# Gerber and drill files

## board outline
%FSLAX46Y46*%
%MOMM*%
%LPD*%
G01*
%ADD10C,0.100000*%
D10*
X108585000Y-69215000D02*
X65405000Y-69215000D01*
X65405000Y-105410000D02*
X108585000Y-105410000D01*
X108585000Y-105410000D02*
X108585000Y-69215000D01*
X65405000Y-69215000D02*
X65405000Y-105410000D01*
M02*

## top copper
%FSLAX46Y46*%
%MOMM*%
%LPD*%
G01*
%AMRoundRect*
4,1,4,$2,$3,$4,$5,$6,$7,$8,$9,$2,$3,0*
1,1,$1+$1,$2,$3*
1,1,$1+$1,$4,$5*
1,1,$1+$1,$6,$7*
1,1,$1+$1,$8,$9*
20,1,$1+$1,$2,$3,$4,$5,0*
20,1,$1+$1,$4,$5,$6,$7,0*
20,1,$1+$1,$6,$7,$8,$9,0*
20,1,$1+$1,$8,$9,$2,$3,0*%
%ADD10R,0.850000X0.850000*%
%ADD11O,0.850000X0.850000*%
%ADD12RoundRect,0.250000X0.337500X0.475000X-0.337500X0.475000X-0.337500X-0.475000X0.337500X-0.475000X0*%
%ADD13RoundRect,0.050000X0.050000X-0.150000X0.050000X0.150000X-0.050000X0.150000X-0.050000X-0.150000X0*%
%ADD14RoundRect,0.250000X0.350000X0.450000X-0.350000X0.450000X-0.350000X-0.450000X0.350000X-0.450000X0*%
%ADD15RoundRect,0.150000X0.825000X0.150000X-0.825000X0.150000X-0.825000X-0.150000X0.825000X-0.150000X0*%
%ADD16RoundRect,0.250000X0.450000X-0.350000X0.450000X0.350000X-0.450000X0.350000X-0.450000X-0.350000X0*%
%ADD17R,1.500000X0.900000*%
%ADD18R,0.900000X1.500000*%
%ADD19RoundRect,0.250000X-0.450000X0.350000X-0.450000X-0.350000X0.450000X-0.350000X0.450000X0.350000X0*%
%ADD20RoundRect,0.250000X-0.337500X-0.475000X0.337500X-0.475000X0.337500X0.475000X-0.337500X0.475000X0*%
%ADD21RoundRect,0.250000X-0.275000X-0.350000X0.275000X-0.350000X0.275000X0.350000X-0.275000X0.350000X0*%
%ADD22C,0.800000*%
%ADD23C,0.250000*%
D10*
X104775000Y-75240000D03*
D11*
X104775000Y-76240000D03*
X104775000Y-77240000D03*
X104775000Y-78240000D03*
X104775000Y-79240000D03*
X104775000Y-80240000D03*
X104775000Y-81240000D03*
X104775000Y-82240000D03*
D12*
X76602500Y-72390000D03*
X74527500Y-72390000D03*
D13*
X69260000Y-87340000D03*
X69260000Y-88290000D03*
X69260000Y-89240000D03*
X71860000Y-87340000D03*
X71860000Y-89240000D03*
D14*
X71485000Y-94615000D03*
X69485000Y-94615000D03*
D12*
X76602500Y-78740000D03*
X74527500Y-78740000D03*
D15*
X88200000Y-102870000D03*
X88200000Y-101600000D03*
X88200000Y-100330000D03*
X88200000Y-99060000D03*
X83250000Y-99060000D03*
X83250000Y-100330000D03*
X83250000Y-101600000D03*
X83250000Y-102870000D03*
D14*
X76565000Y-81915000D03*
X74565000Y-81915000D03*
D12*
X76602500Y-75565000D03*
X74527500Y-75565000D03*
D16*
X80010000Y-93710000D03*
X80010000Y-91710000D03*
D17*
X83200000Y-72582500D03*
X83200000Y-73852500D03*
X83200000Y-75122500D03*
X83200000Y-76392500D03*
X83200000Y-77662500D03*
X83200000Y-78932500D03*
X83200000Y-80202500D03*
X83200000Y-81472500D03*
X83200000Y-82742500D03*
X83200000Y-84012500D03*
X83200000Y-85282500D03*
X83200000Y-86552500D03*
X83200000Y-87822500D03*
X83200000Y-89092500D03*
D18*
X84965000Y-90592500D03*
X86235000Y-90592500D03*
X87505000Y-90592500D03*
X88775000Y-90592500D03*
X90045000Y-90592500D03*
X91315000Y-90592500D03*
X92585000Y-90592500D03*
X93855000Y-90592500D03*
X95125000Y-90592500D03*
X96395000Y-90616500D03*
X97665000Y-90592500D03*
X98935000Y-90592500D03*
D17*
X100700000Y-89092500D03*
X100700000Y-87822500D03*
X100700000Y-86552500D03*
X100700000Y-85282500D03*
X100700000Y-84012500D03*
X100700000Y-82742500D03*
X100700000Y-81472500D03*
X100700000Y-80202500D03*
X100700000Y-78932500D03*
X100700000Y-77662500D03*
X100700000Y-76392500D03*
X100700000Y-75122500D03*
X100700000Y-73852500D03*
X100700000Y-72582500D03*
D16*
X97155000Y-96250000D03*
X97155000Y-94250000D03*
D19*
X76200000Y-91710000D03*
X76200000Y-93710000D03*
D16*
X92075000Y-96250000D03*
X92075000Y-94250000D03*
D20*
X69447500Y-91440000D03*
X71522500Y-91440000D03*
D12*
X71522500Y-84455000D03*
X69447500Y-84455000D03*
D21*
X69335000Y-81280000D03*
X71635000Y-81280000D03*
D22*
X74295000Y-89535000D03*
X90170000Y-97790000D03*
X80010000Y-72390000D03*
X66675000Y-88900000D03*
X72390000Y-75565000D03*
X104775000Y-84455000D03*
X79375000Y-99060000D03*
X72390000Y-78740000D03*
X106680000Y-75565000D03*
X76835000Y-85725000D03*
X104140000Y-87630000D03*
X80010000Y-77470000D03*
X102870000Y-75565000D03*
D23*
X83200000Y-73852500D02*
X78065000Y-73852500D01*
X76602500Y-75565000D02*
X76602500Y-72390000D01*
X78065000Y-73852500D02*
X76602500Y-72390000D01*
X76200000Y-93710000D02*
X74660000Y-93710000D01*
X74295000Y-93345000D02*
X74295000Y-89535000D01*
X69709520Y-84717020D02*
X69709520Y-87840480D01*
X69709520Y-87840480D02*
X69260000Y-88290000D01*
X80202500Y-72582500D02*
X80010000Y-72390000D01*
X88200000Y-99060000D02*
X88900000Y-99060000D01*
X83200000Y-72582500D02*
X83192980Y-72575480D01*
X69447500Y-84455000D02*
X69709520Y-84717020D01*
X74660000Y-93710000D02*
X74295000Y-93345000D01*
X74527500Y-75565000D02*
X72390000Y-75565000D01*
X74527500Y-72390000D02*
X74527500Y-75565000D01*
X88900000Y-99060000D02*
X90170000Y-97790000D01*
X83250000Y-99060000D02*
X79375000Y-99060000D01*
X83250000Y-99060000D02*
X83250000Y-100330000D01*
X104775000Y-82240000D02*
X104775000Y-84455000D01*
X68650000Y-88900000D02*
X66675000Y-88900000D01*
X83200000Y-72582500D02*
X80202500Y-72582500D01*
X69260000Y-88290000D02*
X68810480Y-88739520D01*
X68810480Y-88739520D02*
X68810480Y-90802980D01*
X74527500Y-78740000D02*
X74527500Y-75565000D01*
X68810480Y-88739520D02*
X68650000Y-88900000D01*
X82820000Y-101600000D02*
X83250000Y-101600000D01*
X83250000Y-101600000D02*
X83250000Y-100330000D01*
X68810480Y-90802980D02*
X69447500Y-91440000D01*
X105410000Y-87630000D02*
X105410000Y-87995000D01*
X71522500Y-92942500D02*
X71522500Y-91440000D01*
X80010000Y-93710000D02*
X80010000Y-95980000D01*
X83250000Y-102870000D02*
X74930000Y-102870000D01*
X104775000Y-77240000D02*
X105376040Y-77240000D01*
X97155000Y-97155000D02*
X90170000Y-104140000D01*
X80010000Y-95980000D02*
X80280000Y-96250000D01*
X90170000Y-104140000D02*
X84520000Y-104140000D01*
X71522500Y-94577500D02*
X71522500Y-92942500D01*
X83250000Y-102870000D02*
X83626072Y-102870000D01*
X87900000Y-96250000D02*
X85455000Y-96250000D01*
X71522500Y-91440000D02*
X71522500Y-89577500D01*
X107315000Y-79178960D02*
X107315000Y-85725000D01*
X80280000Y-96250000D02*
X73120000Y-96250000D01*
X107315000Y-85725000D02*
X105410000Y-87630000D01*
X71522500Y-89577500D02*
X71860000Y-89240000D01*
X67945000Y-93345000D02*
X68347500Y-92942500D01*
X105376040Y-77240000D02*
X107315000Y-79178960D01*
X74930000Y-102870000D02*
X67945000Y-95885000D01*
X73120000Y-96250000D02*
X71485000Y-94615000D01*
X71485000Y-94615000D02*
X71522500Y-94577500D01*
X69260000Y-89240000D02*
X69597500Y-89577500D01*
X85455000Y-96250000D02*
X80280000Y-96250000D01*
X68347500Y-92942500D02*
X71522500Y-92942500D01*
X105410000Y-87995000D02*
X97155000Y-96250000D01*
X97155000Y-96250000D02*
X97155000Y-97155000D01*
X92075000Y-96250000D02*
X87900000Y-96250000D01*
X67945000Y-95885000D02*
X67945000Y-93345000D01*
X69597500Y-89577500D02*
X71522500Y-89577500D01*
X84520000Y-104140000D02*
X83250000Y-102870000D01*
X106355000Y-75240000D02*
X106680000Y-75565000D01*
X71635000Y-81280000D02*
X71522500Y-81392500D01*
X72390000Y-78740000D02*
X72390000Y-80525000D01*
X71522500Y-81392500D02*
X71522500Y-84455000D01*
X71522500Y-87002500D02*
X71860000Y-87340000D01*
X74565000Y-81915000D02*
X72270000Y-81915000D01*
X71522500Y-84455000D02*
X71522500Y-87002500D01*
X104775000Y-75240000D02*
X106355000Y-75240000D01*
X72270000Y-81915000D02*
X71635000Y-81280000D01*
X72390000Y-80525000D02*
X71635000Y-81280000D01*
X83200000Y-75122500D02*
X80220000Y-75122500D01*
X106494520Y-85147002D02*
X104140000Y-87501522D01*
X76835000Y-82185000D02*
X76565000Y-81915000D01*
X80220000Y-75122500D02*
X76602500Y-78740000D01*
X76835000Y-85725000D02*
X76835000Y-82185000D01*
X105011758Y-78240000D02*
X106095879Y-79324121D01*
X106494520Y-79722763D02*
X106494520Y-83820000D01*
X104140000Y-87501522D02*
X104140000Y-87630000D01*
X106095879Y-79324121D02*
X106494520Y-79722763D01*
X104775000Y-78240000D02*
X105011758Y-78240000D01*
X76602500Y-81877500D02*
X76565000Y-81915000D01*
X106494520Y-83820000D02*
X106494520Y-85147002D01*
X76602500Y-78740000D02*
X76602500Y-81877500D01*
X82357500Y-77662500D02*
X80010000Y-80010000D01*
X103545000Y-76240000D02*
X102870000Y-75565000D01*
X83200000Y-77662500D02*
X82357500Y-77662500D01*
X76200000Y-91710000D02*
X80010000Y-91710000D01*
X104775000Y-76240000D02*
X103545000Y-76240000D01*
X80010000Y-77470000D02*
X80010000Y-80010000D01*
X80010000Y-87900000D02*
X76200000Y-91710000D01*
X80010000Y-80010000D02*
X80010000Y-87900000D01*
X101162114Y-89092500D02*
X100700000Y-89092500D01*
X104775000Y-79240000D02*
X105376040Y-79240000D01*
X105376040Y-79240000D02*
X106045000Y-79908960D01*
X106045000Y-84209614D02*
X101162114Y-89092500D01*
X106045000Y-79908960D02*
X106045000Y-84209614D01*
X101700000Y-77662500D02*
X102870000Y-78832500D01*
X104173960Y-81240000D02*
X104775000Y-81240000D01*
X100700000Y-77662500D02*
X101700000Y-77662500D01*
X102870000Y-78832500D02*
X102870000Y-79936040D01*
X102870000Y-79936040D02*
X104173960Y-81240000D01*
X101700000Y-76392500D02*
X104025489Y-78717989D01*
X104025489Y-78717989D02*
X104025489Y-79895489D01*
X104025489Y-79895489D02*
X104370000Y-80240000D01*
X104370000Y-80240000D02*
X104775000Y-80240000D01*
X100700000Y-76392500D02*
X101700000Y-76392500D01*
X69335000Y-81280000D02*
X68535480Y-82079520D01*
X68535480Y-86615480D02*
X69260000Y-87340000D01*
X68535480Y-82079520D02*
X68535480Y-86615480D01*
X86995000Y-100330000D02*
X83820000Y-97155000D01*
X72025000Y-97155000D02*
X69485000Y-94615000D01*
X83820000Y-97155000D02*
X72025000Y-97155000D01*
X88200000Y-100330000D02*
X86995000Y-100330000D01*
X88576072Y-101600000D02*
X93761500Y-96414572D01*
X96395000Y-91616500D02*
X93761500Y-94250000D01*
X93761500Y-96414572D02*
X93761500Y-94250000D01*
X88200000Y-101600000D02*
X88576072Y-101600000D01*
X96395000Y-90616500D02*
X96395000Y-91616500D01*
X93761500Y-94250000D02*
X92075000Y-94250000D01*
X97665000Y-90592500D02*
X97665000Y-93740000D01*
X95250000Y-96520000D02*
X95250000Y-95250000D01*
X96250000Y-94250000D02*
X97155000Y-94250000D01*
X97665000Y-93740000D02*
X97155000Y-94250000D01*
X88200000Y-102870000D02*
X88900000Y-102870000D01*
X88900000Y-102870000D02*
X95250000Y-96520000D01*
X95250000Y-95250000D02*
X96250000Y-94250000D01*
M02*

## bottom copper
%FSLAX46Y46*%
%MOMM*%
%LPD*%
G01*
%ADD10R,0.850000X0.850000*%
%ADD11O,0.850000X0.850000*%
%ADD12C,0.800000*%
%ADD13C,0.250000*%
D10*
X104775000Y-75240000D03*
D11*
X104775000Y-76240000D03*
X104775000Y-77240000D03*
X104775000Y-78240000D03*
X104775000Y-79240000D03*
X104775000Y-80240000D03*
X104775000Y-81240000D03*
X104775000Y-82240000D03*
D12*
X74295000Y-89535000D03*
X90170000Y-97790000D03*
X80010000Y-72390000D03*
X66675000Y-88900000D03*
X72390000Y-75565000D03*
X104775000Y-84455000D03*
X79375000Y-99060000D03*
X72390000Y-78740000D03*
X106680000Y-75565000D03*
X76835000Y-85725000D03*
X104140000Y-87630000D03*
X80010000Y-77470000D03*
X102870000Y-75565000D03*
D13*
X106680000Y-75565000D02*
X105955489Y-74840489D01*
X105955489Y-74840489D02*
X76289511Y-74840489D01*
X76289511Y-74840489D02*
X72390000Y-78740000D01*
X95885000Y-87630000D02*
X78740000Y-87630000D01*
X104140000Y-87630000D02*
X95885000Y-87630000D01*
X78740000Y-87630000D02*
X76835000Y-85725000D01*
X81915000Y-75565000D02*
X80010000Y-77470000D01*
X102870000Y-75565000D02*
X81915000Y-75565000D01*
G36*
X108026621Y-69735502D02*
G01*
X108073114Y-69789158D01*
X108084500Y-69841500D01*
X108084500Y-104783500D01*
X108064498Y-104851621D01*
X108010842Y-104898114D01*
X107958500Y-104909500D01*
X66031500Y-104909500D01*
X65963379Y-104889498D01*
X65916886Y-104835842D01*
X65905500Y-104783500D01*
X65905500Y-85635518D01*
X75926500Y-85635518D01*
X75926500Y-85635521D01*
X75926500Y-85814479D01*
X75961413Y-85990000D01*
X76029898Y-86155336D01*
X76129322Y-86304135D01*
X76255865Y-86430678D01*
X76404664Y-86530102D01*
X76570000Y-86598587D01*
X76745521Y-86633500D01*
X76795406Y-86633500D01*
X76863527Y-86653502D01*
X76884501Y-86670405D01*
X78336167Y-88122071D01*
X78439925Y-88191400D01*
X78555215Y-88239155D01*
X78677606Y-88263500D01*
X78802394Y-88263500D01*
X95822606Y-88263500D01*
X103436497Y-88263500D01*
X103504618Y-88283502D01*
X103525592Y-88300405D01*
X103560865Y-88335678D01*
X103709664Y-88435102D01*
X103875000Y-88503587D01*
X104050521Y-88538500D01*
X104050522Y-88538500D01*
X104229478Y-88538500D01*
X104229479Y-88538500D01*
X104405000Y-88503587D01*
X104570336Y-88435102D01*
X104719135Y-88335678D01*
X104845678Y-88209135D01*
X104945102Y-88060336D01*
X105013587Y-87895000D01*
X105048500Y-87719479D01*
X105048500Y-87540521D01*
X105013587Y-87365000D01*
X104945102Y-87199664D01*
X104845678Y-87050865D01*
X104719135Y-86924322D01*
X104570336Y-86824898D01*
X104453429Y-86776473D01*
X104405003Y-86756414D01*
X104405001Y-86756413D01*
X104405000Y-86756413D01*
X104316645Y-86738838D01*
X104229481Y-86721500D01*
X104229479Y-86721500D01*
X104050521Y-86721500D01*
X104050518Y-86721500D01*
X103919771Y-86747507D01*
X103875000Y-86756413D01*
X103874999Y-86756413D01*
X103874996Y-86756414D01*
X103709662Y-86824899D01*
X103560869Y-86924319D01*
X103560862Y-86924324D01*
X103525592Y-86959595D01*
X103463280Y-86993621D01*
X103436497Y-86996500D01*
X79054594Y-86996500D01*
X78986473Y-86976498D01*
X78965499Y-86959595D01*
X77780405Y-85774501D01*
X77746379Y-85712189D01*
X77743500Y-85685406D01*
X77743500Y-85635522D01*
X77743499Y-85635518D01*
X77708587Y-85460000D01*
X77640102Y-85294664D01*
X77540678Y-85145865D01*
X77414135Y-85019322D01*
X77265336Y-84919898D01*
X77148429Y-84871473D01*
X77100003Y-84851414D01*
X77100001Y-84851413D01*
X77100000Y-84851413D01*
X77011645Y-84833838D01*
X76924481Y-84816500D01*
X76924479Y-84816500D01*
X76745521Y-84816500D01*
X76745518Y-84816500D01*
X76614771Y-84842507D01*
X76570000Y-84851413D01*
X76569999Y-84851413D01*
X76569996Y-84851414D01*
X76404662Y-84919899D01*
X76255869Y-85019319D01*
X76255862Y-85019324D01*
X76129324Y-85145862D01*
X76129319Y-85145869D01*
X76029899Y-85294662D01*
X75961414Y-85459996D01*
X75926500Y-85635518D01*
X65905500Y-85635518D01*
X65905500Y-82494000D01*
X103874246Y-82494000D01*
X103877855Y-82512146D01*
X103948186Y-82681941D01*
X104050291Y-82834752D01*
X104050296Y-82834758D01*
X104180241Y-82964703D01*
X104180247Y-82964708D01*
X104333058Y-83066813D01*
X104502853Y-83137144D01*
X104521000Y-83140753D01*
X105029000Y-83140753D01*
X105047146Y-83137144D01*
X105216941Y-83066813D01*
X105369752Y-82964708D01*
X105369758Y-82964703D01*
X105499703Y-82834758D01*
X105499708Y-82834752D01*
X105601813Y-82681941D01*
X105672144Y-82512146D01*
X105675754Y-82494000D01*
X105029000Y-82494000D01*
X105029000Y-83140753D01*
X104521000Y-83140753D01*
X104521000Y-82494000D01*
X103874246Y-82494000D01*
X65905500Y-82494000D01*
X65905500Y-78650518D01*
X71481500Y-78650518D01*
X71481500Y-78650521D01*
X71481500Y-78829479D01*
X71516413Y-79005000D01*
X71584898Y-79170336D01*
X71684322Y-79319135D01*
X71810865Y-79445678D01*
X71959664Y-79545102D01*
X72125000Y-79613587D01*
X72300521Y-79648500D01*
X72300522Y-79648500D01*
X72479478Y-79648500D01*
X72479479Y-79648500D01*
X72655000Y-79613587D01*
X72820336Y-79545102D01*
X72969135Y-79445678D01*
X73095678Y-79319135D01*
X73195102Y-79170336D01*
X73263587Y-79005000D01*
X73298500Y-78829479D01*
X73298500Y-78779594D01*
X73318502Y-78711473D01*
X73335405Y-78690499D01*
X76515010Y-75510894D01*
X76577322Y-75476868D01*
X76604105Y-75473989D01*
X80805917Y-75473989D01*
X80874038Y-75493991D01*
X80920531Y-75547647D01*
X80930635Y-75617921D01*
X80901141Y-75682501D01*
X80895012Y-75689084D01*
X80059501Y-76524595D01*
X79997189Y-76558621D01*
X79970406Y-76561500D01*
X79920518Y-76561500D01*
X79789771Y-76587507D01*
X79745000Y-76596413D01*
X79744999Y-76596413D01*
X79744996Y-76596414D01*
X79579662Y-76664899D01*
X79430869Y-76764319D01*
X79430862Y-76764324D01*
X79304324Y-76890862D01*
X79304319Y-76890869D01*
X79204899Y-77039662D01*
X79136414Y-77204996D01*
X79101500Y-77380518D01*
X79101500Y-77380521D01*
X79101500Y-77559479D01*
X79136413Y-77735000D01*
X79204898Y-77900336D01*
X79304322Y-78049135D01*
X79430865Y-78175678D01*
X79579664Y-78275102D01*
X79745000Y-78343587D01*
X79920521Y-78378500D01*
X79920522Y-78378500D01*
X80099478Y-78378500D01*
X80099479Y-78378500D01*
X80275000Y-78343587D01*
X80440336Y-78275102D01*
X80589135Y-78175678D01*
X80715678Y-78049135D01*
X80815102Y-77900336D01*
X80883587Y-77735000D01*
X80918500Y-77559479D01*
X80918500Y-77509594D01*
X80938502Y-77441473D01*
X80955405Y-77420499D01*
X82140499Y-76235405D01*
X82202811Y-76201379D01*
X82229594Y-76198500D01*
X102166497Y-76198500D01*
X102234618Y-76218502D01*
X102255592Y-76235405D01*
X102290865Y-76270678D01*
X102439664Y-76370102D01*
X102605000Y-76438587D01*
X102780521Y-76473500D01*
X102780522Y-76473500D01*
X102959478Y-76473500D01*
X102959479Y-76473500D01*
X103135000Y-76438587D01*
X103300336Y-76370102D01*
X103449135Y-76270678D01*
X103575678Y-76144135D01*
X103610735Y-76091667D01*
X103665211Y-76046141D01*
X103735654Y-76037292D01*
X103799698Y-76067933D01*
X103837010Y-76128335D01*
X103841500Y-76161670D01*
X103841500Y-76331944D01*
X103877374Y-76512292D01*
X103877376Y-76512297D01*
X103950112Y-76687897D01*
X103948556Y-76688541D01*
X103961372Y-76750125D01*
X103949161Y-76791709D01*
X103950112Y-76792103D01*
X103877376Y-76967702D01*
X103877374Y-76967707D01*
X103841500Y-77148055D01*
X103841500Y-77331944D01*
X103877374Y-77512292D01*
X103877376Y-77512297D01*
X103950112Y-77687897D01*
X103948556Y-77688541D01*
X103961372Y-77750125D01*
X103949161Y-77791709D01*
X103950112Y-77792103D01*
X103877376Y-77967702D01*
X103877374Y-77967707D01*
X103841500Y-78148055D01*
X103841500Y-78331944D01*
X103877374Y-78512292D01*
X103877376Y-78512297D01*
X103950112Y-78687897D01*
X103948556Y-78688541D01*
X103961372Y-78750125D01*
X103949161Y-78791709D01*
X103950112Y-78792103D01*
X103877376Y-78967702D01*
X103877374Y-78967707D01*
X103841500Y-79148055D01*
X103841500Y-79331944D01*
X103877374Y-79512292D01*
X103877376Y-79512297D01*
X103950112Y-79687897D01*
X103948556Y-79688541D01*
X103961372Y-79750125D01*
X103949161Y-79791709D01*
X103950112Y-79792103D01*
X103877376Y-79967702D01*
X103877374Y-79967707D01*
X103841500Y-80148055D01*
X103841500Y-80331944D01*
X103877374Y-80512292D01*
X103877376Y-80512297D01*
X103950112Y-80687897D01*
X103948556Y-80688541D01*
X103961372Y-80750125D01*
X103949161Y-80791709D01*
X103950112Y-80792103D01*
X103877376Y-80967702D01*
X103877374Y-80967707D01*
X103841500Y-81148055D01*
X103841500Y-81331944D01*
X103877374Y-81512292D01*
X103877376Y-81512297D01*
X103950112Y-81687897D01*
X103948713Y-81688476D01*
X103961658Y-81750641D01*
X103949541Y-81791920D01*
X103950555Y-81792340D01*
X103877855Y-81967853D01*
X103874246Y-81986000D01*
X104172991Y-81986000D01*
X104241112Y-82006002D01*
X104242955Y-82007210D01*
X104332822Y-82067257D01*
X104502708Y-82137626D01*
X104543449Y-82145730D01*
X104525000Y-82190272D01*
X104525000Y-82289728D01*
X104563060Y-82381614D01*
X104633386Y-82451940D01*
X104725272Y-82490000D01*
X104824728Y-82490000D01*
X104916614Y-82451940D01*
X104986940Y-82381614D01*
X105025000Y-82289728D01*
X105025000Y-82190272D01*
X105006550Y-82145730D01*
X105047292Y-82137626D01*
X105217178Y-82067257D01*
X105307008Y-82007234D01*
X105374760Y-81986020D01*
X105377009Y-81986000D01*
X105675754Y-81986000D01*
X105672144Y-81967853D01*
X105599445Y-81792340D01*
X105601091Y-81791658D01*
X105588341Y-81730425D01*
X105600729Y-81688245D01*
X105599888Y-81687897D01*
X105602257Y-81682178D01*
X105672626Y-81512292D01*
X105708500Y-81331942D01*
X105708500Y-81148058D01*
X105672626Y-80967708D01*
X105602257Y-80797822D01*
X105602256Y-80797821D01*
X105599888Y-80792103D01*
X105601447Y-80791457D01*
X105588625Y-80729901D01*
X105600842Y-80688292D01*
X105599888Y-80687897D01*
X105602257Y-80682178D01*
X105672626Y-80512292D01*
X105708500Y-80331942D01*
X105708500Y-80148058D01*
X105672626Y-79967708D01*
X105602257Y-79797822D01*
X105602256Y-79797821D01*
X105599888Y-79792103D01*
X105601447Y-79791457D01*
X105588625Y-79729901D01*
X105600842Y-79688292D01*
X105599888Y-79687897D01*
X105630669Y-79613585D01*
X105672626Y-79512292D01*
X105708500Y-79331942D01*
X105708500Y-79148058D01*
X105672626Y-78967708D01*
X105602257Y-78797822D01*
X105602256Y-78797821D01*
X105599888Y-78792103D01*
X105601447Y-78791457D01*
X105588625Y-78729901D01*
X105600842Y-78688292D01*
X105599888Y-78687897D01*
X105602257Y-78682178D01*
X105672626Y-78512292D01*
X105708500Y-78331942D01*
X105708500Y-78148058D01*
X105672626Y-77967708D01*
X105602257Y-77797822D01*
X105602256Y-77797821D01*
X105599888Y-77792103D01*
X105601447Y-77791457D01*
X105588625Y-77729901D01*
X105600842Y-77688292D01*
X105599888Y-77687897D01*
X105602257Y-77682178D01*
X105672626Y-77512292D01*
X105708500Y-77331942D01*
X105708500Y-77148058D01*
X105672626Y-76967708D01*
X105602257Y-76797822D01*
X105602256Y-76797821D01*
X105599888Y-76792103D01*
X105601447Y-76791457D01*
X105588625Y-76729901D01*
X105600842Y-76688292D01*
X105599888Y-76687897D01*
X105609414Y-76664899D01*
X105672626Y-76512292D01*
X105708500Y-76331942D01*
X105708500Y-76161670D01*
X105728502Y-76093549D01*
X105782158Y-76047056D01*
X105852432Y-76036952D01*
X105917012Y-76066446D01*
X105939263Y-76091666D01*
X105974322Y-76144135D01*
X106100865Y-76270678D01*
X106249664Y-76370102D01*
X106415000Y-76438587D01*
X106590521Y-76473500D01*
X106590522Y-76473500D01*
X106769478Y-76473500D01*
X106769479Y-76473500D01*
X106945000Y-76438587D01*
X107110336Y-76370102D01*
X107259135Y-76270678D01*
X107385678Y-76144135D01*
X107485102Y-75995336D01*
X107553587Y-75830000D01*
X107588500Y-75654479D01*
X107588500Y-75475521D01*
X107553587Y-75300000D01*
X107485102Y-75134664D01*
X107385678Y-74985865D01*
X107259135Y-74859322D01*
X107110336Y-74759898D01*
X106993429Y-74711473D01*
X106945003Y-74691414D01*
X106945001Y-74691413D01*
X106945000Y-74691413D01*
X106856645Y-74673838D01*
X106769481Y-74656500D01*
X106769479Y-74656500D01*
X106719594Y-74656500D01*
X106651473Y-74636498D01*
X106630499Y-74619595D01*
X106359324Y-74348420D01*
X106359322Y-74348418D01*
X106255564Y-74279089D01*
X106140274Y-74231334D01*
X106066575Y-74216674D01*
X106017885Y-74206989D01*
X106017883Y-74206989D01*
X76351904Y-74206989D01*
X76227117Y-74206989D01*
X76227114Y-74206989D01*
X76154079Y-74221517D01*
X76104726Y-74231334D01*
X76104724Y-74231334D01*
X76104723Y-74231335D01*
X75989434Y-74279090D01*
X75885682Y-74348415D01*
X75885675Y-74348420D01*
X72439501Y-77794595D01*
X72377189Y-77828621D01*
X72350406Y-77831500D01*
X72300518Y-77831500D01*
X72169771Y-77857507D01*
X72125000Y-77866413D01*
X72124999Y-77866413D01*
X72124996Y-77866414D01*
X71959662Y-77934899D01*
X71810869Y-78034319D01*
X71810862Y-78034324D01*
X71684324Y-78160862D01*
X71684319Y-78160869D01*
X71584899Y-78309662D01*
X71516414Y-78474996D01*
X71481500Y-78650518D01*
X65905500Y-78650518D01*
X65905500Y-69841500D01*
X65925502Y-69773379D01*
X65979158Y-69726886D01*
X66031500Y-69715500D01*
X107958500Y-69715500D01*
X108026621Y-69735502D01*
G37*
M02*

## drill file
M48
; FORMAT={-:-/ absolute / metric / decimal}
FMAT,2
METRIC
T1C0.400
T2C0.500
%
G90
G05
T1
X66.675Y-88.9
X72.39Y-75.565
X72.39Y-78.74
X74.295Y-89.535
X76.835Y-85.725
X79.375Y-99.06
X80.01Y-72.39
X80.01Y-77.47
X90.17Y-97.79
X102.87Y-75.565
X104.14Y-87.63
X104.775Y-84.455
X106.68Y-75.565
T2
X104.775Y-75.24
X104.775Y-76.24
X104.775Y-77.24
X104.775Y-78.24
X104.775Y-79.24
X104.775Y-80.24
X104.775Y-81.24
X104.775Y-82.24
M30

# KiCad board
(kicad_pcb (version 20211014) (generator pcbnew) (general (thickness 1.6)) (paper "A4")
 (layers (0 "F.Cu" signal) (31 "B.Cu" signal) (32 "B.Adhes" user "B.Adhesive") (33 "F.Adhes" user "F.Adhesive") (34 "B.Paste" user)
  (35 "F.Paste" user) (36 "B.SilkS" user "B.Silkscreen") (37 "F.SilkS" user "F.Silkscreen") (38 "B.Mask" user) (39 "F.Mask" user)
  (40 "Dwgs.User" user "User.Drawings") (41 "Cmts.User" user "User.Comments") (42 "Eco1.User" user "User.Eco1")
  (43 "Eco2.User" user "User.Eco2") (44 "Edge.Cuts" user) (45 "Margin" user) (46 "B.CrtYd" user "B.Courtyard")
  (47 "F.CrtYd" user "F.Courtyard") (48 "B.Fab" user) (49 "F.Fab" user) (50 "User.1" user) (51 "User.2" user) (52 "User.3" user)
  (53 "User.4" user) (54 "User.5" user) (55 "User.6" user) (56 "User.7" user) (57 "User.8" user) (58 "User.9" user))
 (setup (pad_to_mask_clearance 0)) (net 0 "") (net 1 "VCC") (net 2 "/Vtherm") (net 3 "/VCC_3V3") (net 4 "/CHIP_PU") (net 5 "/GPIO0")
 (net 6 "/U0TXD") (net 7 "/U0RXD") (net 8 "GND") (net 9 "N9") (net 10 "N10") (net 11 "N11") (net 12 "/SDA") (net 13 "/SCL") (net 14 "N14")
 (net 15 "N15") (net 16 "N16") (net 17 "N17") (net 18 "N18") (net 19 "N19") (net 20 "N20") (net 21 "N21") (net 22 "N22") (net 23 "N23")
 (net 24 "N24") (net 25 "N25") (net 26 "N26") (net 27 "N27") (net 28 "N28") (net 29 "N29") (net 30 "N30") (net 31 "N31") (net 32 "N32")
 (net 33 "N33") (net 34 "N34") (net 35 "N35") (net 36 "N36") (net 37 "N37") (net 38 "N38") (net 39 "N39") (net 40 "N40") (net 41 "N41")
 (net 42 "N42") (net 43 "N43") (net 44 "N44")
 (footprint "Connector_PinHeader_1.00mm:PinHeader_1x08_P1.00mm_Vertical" (layer "F.Cu") (at 104.775 75.24)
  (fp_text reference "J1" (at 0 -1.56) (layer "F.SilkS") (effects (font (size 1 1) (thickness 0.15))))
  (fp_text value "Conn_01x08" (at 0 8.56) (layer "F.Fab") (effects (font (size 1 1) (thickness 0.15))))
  (pad "1" thru_hole rect (at 0 0) (size 0.85 0.85) (drill 0.5) (layers *.Cu *.Mask) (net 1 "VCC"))
  (pad "2" thru_hole oval (at 0 1) (size 0.85 0.85) (drill 0.5) (layers *.Cu *.Mask) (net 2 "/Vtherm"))
  (pad "3" thru_hole oval (at 0 2) (size 0.85 0.85) (drill 0.5) (layers *.Cu *.Mask) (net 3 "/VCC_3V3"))
  (pad "4" thru_hole oval (at 0 3) (size 0.85 0.85) (drill 0.5) (layers *.Cu *.Mask) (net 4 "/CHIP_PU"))
  (pad "5" thru_hole oval (at 0 4) (size 0.85 0.85) (drill 0.5) (layers *.Cu *.Mask) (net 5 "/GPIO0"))
  (pad "6" thru_hole oval (at 0 5) (size 0.85 0.85) (drill 0.5) (layers *.Cu *.Mask) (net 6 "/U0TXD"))
  (pad "7" thru_hole oval (at 0 6) (size 0.85 0.85) (drill 0.5) (layers *.Cu *.Mask) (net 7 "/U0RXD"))
  (pad "8" thru_hole oval (at 0 7) (size 0.85 0.85) (drill 0.5) (layers *.Cu *.Mask) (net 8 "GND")))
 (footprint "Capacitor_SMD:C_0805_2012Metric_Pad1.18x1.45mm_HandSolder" (layer "F.Cu") (at 75.565 72.39 180)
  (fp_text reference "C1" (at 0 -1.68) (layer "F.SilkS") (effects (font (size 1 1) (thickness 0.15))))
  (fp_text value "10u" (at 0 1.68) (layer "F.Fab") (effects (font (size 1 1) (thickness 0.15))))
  (pad "1" smd roundrect (at -1.0375 0 180) (size 1.175 1.45) (layers "F.Cu" "F.Paste" "F.Mask") (roundrect_rratio 0.212766) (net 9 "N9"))
  (pad "2" smd roundrect (at 1.0375 0 180) (size 1.175 1.45) (layers "F.Cu" "F.Paste" "F.Mask") (roundrect_rratio 0.212766) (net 8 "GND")))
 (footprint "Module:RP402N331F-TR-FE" (layer "F.Cu") (at 69.26 87.34)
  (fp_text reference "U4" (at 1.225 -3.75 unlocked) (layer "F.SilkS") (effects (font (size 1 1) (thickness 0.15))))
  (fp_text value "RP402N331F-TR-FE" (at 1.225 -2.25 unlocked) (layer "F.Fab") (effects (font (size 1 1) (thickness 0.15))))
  (pad "1" smd roundrect (at 0 0 90) (size 0.4 0.2) (layers "F.Cu" "F.Paste" "F.Mask") (roundrect_rratio 0.25) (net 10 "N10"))
  (pad "2" smd roundrect (at 0 0.95 90) (size 0.4 0.2) (layers "F.Cu" "F.Paste" "F.Mask") (roundrect_rratio 0.25) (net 8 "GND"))
  (pad "3" smd roundrect (at 0 1.9 90) (size 0.4 0.2) (layers "F.Cu" "F.Paste" "F.Mask") (roundrect_rratio 0.25) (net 3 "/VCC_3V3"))
  (pad "4" smd roundrect (at 2.6 0 90) (size 0.4 0.2) (layers "F.Cu" "F.Paste" "F.Mask") (roundrect_rratio 0.25) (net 1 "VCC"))
  (pad "5" smd roundrect (at 2.6 1.9 90) (size 0.4 0.2) (layers "F.Cu" "F.Paste" "F.Mask") (roundrect_rratio 0.25) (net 3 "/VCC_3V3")))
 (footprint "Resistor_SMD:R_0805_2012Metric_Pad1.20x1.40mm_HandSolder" (layer "F.Cu") (at 70.485 94.615 180)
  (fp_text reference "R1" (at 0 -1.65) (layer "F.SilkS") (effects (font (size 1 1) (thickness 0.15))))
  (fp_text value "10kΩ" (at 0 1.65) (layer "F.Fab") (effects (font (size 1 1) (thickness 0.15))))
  (pad "1" smd roundrect (at -1 0 180) (size 1.2 1.4) (layers "F.Cu" "F.Paste" "F.Mask") (roundrect_rratio 0.208333) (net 3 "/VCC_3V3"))
  (pad "2" smd roundrect (at 1 0 180) (size 1.2 1.4) (layers "F.Cu" "F.Paste" "F.Mask") (roundrect_rratio 0.208333) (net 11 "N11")))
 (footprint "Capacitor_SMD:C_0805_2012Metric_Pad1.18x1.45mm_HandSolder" (layer "F.Cu") (at 75.565 78.74 180)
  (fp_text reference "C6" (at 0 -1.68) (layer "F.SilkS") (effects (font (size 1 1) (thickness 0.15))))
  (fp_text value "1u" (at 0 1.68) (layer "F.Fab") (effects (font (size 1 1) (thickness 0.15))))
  (pad "1" smd roundrect (at -1.0375 0 180) (size 1.175 1.45) (layers "F.Cu" "F.Paste" "F.Mask") (roundrect_rratio 0.212766)
   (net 4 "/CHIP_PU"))
  (pad "2" smd roundrect (at 1.0375 0 180) (size 1.175 1.45) (layers "F.Cu" "F.Paste" "F.Mask") (roundrect_rratio 0.212766) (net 8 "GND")))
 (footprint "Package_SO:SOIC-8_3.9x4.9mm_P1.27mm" (layer "F.Cu") (at 85.725 100.965 180)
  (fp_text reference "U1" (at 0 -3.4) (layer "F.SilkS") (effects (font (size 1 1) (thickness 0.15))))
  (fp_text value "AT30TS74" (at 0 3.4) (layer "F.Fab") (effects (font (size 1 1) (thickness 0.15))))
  (pad "1" smd roundrect (at -2.475 -1.905 180) (size 1.95 0.6) (layers "F.Cu" "F.Paste" "F.Mask") (roundrect_rratio 0.25) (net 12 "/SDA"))
  (pad "2" smd roundrect (at -2.475 -0.635 180) (size 1.95 0.6) (layers "F.Cu" "F.Paste" "F.Mask") (roundrect_rratio 0.25) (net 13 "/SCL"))
  (pad "3" smd roundrect (at -2.475 0.635 180) (size 1.95 0.6) (layers "F.Cu" "F.Paste" "F.Mask") (roundrect_rratio 0.25) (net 11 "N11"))
  (pad "4" smd roundrect (at -2.475 1.905 180) (size 1.95 0.6) (layers "F.Cu" "F.Paste" "F.Mask") (roundrect_rratio 0.25) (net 8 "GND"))
  (pad "5" smd roundrect (at 2.475 1.905 180) (size 1.95 0.6) (layers "F.Cu" "F.Paste" "F.Mask") (roundrect_rratio 0.25) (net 8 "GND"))
  (pad "6" smd roundrect (at 2.475 0.635 180) (size 1.95 0.6) (layers "F.Cu" "F.Paste" "F.Mask") (roundrect_rratio 0.25) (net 8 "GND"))
  (pad "7" smd roundrect (at 2.475 -0.635 180) (size 1.95 0.6) (layers "F.Cu" "F.Paste" "F.Mask") (roundrect_rratio 0.25) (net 8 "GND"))
  (pad "8" smd roundrect (at 2.475 -1.905 180) (size 1.95 0.6) (layers "F.Cu" "F.Paste" "F.Mask") (roundrect_rratio 0.25) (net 3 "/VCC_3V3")))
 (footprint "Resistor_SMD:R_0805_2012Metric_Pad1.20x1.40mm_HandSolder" (layer "F.Cu") (at 75.565 81.915 180)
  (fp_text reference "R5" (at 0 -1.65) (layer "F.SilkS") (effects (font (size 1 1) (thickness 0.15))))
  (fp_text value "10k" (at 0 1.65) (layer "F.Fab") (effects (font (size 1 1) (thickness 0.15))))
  (pad "1" smd roundrect (at -1 0 180) (size 1.2 1.4) (layers "F.Cu" "F.Paste" "F.Mask") (roundrect_rratio 0.208333) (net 4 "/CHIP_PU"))
  (pad "2" smd roundrect (at 1 0 180) (size 1.2 1.4) (layers "F.Cu" "F.Paste" "F.Mask") (roundrect_rratio 0.208333) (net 1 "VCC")))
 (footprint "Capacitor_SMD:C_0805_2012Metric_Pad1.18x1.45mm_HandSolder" (layer "F.Cu") (at 75.565 75.565 180)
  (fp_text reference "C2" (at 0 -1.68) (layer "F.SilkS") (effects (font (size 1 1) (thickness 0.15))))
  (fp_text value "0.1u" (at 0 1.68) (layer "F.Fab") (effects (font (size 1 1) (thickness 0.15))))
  (pad "1" smd roundrect (at -1.0375 0 180) (size 1.175 1.45) (layers "F.Cu" "F.Paste" "F.Mask") (roundrect_rratio 0.212766) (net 9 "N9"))
  (pad "2" smd roundrect (at 1.0375 0 180) (size 1.175 1.45) (layers "F.Cu" "F.Paste" "F.Mask") (roundrect_rratio 0.212766) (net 8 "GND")))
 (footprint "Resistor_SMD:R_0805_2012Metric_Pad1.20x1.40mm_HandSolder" (layer "F.Cu") (at 80.01 92.71 90)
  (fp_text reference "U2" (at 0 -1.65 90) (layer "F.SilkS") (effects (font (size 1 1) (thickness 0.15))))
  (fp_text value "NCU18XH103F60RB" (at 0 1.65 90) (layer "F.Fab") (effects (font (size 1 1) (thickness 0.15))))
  (pad "1" smd roundrect (at -1 0 90) (size 1.2 1.4) (layers "F.Cu" "F.Paste" "F.Mask") (roundrect_rratio 0.208333) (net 3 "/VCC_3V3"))
  (pad "2" smd roundrect (at 1 0 90) (size 1.2 1.4) (layers "F.Cu" "F.Paste" "F.Mask") (roundrect_rratio 0.208333) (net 2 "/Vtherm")))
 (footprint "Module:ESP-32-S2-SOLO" (layer "F.Cu") (at 83.2 72.5825)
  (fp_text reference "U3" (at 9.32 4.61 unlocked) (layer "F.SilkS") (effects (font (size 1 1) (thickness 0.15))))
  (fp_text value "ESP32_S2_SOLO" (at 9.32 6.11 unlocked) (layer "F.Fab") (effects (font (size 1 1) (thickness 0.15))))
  (pad "1" smd rect (at 0 0) (size 1.5 0.9) (layers "F.Cu" "F.Paste" "F.Mask") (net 8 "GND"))
  (pad "2" smd rect (at 0 1.27) (size 1.5 0.9) (layers "F.Cu" "F.Paste" "F.Mask") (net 9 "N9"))
  (pad "3" smd rect (at 0 2.54) (size 1.5 0.9) (layers "F.Cu" "F.Paste" "F.Mask") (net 4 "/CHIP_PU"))
  (pad "4" smd rect (at 0 3.81) (size 1.5 0.9) (layers "F.Cu" "F.Paste" "F.Mask") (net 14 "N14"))
  (pad "5" smd rect (at 0 5.08) (size 1.5 0.9) (layers "F.Cu" "F.Paste" "F.Mask") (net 2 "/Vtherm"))
  (pad "6" smd rect (at 0 6.35) (size 1.5 0.9) (layers "F.Cu" "F.Paste" "F.Mask") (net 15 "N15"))
  (pad "7" smd rect (at 0 7.62) (size 1.5 0.9) (layers "F.Cu" "F.Paste" "F.Mask") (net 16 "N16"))
  (pad "8" smd rect (at 0 8.89) (size 1.5 0.9) (layers "F.Cu" "F.Paste" "F.Mask") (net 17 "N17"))
  (pad "9" smd rect (at 0 10.16) (size 1.5 0.9) (layers "F.Cu" "F.Paste" "F.Mask") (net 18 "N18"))
  (pad "10" smd rect (at 0 11.43) (size 1.5 0.9) (layers "F.Cu" "F.Paste" "F.Mask") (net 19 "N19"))
  (pad "11" smd rect (at 0 12.7) (size 1.5 0.9) (layers "F.Cu" "F.Paste" "F.Mask") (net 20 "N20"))
  (pad "12" smd rect (at 0 13.97) (size 1.5 0.9) (layers "F.Cu" "F.Paste" "F.Mask") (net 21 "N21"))
  (pad "13" smd rect (at 0 15.24) (size 1.5 0.9) (layers "F.Cu" "F.Paste" "F.Mask") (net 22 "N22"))
  (pad "14" smd rect (at 0 16.51) (size 1.5 0.9) (layers "F.Cu" "F.Paste" "F.Mask") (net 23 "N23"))
  (pad "15" smd rect (at 1.765 18.01 90) (size 1.5 0.9) (layers "F.Cu" "F.Paste" "F.Mask") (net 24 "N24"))
  (pad "16" smd rect (at 3.035 18.01 90) (size 1.5 0.9) (layers "F.Cu" "F.Paste" "F.Mask") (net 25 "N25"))
  (pad "17" smd rect (at 4.305 18.01 90) (size 1.5 0.9) (layers "F.Cu" "F.Paste" "F.Mask") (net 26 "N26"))
  (pad "18" smd rect (at 5.575 18.01 90) (size 1.5 0.9) (layers "F.Cu" "F.Paste" "F.Mask") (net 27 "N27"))
  (pad "19" smd rect (at 6.845 18.01 90) (size 1.5 0.9) (layers "F.Cu" "F.Paste" "F.Mask") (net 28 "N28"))
  (pad "20" smd rect (at 8.115 18.01 90) (size 1.5 0.9) (layers "F.Cu" "F.Paste" "F.Mask") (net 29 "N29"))
  (pad "21" smd rect (at 9.385 18.01 90) (size 1.5 0.9) (layers "F.Cu" "F.Paste" "F.Mask") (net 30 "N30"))
  (pad "22" smd rect (at 10.655 18.01 90) (size 1.5 0.9) (layers "F.Cu" "F.Paste" "F.Mask") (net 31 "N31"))
  (pad "23" smd rect (at 11.925 18.01 90) (size 1.5 0.9) (layers "F.Cu" "F.Paste" "F.Mask") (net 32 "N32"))
  (pad "24" smd rect (at 13.195 18.034 90) (size 1.5 0.9) (layers "F.Cu" "F.Paste" "F.Mask") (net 13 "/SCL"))
  (pad "25" smd rect (at 14.465 18.01 90) (size 1.5 0.9) (layers "F.Cu" "F.Paste" "F.Mask") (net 12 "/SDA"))
  (pad "26" smd rect (at 15.735 18.01 90) (size 1.5 0.9) (layers "F.Cu" "F.Paste" "F.Mask") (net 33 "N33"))
  (pad "27" smd rect (at 17.5 16.51) (size 1.5 0.9) (layers "F.Cu" "F.Paste" "F.Mask") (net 5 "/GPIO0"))
  (pad "28" smd rect (at 17.5 15.24) (size 1.5 0.9) (layers "F.Cu" "F.Paste" "F.Mask") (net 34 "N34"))
  (pad "29" smd rect (at 17.5 13.97) (size 1.5 0.9) (layers "F.Cu" "F.Paste" "F.Mask") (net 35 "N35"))
  (pad "30" smd rect (at 17.5 12.7) (size 1.5 0.9) (layers "F.Cu" "F.Paste" "F.Mask") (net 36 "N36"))
  (pad "31" smd rect (at 17.5 11.43) (size 1.5 0.9) (layers "F.Cu" "F.Paste" "F.Mask") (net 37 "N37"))
  (pad "32" smd rect (at 17.5 10.16) (size 1.5 0.9) (layers "F.Cu" "F.Paste" "F.Mask") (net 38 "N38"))
  (pad "33" smd rect (at 17.5 8.89) (size 1.5 0.9) (layers "F.Cu" "F.Paste" "F.Mask") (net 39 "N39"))
  (pad "34" smd rect (at 17.5 7.62) (size 1.5 0.9) (layers "F.Cu" "F.Paste" "F.Mask") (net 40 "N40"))
  (pad "35" smd rect (at 17.5 6.35) (size 1.5 0.9) (layers "F.Cu" "F.Paste" "F.Mask") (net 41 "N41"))
  (pad "36" smd rect (at 17.5 5.08) (size 1.5 0.9) (layers "F.Cu" "F.Paste" "F.Mask") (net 7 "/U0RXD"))
  (pad "37" smd rect (at 17.5 3.81) (size 1.5 0.9) (layers "F.Cu" "F.Paste" "F.Mask") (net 6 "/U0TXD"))
  (pad "38" smd rect (at 17.5 2.54) (size 1.5 0.9) (layers "F.Cu" "F.Paste" "F.Mask") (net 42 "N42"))
  (pad "39" smd rect (at 17.5 1.27) (size 1.5 0.9) (layers "F.Cu" "F.Paste" "F.Mask") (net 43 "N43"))
  (pad "40" smd rect (at 17.5 0) (size 1.5 0.9) (layers "F.Cu" "F.Paste" "F.Mask") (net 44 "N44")))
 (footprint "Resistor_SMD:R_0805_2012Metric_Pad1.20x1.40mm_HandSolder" (layer "F.Cu") (at 97.155 95.25 90)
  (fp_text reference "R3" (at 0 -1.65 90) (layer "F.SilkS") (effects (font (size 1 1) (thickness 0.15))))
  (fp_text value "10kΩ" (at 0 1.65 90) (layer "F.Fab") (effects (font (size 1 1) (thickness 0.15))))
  (pad "1" smd roundrect (at -1 0 90) (size 1.2 1.4) (layers "F.Cu" "F.Paste" "F.Mask") (roundrect_rratio 0.208333) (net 3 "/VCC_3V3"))
  (pad "2" smd roundrect (at 1 0 90) (size 1.2 1.4) (layers "F.Cu" "F.Paste" "F.Mask") (roundrect_rratio 0.208333) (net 12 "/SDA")))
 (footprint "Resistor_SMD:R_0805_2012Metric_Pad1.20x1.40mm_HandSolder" (layer "F.Cu") (at 76.2 92.71 -90)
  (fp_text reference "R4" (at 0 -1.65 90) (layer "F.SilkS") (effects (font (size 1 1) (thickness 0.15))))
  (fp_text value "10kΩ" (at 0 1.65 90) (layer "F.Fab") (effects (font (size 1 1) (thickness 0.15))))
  (pad "1" smd roundrect (at -1 0 270) (size 1.2 1.4) (layers "F.Cu" "F.Paste" "F.Mask") (roundrect_rratio 0.208333) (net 2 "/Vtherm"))
  (pad "2" smd roundrect (at 1 0 270) (size 1.2 1.4) (layers "F.Cu" "F.Paste" "F.Mask") (roundrect_rratio 0.208333) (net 8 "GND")))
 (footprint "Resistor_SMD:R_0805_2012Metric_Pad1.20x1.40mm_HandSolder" (layer "F.Cu") (at 92.075 95.25 90)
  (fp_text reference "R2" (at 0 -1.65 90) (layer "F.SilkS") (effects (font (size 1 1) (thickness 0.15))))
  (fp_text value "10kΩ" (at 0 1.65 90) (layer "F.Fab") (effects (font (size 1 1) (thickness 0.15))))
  (pad "1" smd roundrect (at -1 0 90) (size 1.2 1.4) (layers "F.Cu" "F.Paste" "F.Mask") (roundrect_rratio 0.208333) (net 3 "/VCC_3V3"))
  (pad "2" smd roundrect (at 1 0 90) (size 1.2 1.4) (layers "F.Cu" "F.Paste" "F.Mask") (roundrect_rratio 0.208333) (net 13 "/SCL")))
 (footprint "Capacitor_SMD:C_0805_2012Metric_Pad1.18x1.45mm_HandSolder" (layer "F.Cu") (at 70.485 91.44)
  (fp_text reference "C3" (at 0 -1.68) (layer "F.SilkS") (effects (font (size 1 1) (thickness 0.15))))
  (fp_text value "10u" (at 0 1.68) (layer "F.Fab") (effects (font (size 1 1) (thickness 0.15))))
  (pad "1" smd roundrect (at -1.0375 0) (size 1.175 1.45) (layers "F.Cu" "F.Paste" "F.Mask") (roundrect_rratio 0.212766) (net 8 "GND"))
  (pad "2" smd roundrect (at 1.0375 0) (size 1.175 1.45) (layers "F.Cu" "F.Paste" "F.Mask") (roundrect_rratio 0.212766) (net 3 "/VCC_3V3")))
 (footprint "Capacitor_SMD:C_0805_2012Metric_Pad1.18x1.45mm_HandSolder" (layer "F.Cu") (at 70.485 84.455 180)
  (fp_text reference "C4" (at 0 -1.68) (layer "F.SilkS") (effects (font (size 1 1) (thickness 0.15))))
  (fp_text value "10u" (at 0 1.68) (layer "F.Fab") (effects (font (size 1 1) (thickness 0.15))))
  (pad "1" smd roundrect (at -1.0375 0 180) (size 1.175 1.45) (layers "F.Cu" "F.Paste" "F.Mask") (roundrect_rratio 0.212766) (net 1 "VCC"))
  (pad "2" smd roundrect (at 1.0375 0 180) (size 1.175 1.45) (layers "F.Cu" "F.Paste" "F.Mask") (roundrect_rratio 0.212766) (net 8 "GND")))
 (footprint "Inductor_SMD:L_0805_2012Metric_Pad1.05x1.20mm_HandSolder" (layer "F.Cu") (at 70.485 81.28)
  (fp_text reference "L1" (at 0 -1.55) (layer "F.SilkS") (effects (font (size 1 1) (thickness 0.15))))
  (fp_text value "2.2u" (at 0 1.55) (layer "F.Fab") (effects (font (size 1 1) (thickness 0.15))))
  (pad "1" smd roundrect (at -1.15 0) (size 1.05 1.2) (layers "F.Cu" "F.Paste" "F.Mask") (roundrect_rratio 0.238095) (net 10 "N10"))
  (pad "2" smd roundrect (at 1.15 0) (size 1.05 1.2) (layers "F.Cu" "F.Paste" "F.Mask") (roundrect_rratio 0.238095) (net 1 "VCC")))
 (gr_line (start 108.585 69.215) (end 65.405 69.215) (layer "Edge.Cuts") (width 0.1))
 (gr_line (start 65.405 105.41) (end 108.585 105.41) (layer "Edge.Cuts") (width 0.1))
 (gr_line (start 108.585 105.41) (end 108.585 69.215) (layer "Edge.Cuts") (width 0.1))
 (gr_line (start 65.405 69.215) (end 65.405 105.41) (layer "Edge.Cuts") (width 0.1))
 (segment (start 83.2 73.8525) (end 78.065 73.8525) (width 0.25) (layer "F.Cu") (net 9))
 (segment (start 76.6025 75.565) (end 76.6025 72.39) (width 0.25) (layer "F.Cu") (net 9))
 (segment (start 78.065 73.8525) (end 76.6025 72.39) (width 0.25) (layer "F.Cu") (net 9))
 (segment (start 76.2 93.71) (end 74.66 93.71) (width 0.25) (layer "F.Cu") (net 8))
 (segment (start 74.295 93.345) (end 74.295 89.535) (width 0.25) (layer "F.Cu") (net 8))
 (segment (start 69.70952 84.71702) (end 69.70952 87.84048) (width 0.25) (layer "F.Cu") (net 8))
 (segment (start 69.70952 87.84048) (end 69.26 88.29) (width 0.25) (layer "F.Cu") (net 8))
 (segment (start 80.2025 72.5825) (end 80.01 72.39) (width 0.25) (layer "F.Cu") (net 8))
 (segment (start 88.2 99.06) (end 88.9 99.06) (width 0.25) (layer "F.Cu") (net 8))
 (segment (start 83.2 72.5825) (end 83.19298 72.57548) (width 0.25) (layer "F.Cu") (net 8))
 (segment (start 69.4475 84.455) (end 69.70952 84.71702) (width 0.25) (layer "F.Cu") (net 8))
 (segment (start 74.66 93.71) (end 74.295 93.345) (width 0.25) (layer "F.Cu") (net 8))
 (segment (start 74.5275 75.565) (end 72.39 75.565) (width 0.25) (layer "F.Cu") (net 8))
 (segment (start 74.5275 72.39) (end 74.5275 75.565) (width 0.25) (layer "F.Cu") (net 8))
 (segment (start 88.9 99.06) (end 90.17 97.79) (width 0.25) (layer "F.Cu") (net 8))
 (segment (start 83.25 99.06) (end 79.375 99.06) (width 0.25) (layer "F.Cu") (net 8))
 (segment (start 83.25 99.06) (end 83.25 100.33) (width 0.25) (layer "F.Cu") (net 8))
 (segment (start 104.775 82.24) (end 104.775 84.455) (width 0.25) (layer "F.Cu") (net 8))
 (segment (start 68.65 88.9) (end 66.675 88.9) (width 0.25) (layer "F.Cu") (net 8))
 (segment (start 83.2 72.5825) (end 80.2025 72.5825) (width 0.25) (layer "F.Cu") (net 8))
 (segment (start 69.26 88.29) (end 68.81048 88.73952) (width 0.25) (layer "F.Cu") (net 8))
 (segment (start 68.81048 88.73952) (end 68.81048 90.80298) (width 0.25) (layer "F.Cu") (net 8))
 (segment (start 74.5275 78.74) (end 74.5275 75.565) (width 0.25) (layer "F.Cu") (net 8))
 (segment (start 68.81048 88.73952) (end 68.65 88.9) (width 0.25) (layer "F.Cu") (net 8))
 (segment (start 82.82 101.6) (end 83.25 101.6) (width 0.25) (layer "F.Cu") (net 8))
 (segment (start 83.25 101.6) (end 83.25 100.33) (width 0.25) (layer "F.Cu") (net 8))
 (segment (start 68.81048 90.80298) (end 69.4475 91.44) (width 0.25) (layer "F.Cu") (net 8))
 (via (at 74.295 89.535) (size 0.8) (drill 0.4) (layers "F.Cu" "B.Cu") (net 8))
 (via (at 90.17 97.79) (size 0.8) (drill 0.4) (layers "F.Cu" "B.Cu") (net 8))
 (via (at 80.01 72.39) (size 0.8) (drill 0.4) (layers "F.Cu" "B.Cu") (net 8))
 (via (at 66.675 88.9) (size 0.8) (drill 0.4) (layers "F.Cu" "B.Cu") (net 8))
 (via (at 72.39 75.565) (size 0.8) (drill 0.4) (layers "F.Cu" "B.Cu") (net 8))
 (via (at 104.775 84.455) (size 0.8) (drill 0.4) (layers "F.Cu" "B.Cu") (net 8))
 (via (at 79.375 99.06) (size 0.8) (drill 0.4) (layers "F.Cu" "B.Cu") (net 8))
 (segment (start 105.41 87.63) (end 105.41 87.995) (width 0.25) (layer "F.Cu") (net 3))
 (segment (start 71.5225 92.9425) (end 71.5225 91.44) (width 0.25) (layer "F.Cu") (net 3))
 (segment (start 80.01 93.71) (end 80.01 95.98) (width 0.25) (layer "F.Cu") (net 3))
 (segment (start 83.25 102.87) (end 74.93 102.87) (width 0.25) (layer "F.Cu") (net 3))
 (segment (start 104.775 77.24) (end 105.37604 77.24) (width 0.25) (layer "F.Cu") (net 3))
 (segment (start 97.155 97.155) (end 90.17 104.14) (width 0.25) (layer "F.Cu") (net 3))
 (segment (start 80.01 95.98) (end 80.28 96.25) (width 0.25) (layer "F.Cu") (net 3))
 (segment (start 90.17 104.14) (end 84.52 104.14) (width 0.25) (layer "F.Cu") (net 3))
 (segment (start 71.5225 94.5775) (end 71.5225 92.9425) (width 0.25) (layer "F.Cu") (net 3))
 (segment (start 83.25 102.87) (end 83.626072 102.87) (width 0.25) (layer "F.Cu") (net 3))
 (segment (start 87.9 96.25) (end 85.455 96.25) (width 0.25) (layer "F.Cu") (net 3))
 (segment (start 71.5225 91.44) (end 71.5225 89.5775) (width 0.25) (layer "F.Cu") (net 3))
 (segment (start 107.315 79.17896) (end 107.315 85.725) (width 0.25) (layer "F.Cu") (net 3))
 (segment (start 80.28 96.25) (end 73.12 96.25) (width 0.25) (layer "F.Cu") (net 3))
 (segment (start 107.315 85.725) (end 105.41 87.63) (width 0.25) (layer "F.Cu") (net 3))
 (segment (start 71.5225 89.5775) (end 71.86 89.24) (width 0.25) (layer "F.Cu") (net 3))
 (segment (start 67.945 93.345) (end 68.3475 92.9425) (width 0.25) (layer "F.Cu") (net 3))
 (segment (start 105.37604 77.24) (end 107.315 79.17896) (width 0.25) (layer "F.Cu") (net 3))
 (segment (start 74.93 102.87) (end 67.945 95.885) (width 0.25) (layer "F.Cu") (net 3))
 (segment (start 73.12 96.25) (end 71.485 94.615) (width 0.25) (layer "F.Cu") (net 3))
 (segment (start 71.485 94.615) (end 71.5225 94.5775) (width 0.25) (layer "F.Cu") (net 3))
 (segment (start 69.26 89.24) (end 69.5975 89.5775) (width 0.25) (layer "F.Cu") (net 3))
 (segment (start 85.455 96.25) (end 80.28 96.25) (width 0.25) (layer "F.Cu") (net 3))
 (segment (start 68.3475 92.9425) (end 71.5225 92.9425) (width 0.25) (layer "F.Cu") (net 3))
 (segment (start 105.41 87.995) (end 97.155 96.25) (width 0.25) (layer "F.Cu") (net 3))
 (segment (start 97.155 96.25) (end 97.155 97.155) (width 0.25) (layer "F.Cu") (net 3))
 (segment (start 92.075 96.25) (end 87.9 96.25) (width 0.25) (layer "F.Cu") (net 3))
 (segment (start 67.945 95.885) (end 67.945 93.345) (width 0.25) (layer "F.Cu") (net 3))
 (segment (start 69.5975 89.5775) (end 71.5225 89.5775) (width 0.25) (layer "F.Cu") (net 3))
 (segment (start 84.52 104.14) (end 83.25 102.87) (width 0.25) (layer "F.Cu") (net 3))
 (segment (start 106.355 75.24) (end 106.68 75.565) (width 0.25) (layer "F.Cu") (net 1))
 (segment (start 71.635 81.28) (end 71.5225 81.3925) (width 0.25) (layer "F.Cu") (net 1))
 (segment (start 72.39 78.74) (end 72.39 80.525) (width 0.25) (layer "F.Cu") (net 1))
 (segment (start 71.5225 81.3925) (end 71.5225 84.455) (width 0.25) (layer "F.Cu") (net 1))
 (segment (start 71.5225 87.0025) (end 71.86 87.34) (width 0.25) (layer "F.Cu") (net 1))
 (segment (start 74.565 81.915) (end 72.27 81.915) (width 0.25) (layer "F.Cu") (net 1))
 (segment (start 71.5225 84.455) (end 71.5225 87.0025) (width 0.25) (layer "F.Cu") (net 1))
 (segment (start 104.775 75.24) (end 106.355 75.24) (width 0.25) (layer "F.Cu") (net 1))
 (segment (start 72.27 81.915) (end 71.635 81.28) (width 0.25) (layer "F.Cu") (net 1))
 (segment (start 72.39 80.525) (end 71.635 81.28) (width 0.25) (layer "F.Cu") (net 1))
 (via (at 72.39 78.74) (size 0.8) (drill 0.4) (layers "F.Cu" "B.Cu") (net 1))
 (via (at 106.68 75.565) (size 0.8) (drill 0.4) (layers "F.Cu" "B.Cu") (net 1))
 (segment (start 106.68 75.565) (end 105.955489 74.840489) (width 0.25) (layer "B.Cu") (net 1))
 (segment (start 105.955489 74.840489) (end 76.289511 74.840489) (width 0.25) (layer "B.Cu") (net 1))
 (segment (start 76.289511 74.840489) (end 72.39 78.74) (width 0.25) (layer "B.Cu") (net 1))
 (segment (start 83.2 75.1225) (end 80.22 75.1225) (width 0.25) (layer "F.Cu") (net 4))
 (segment (start 106.49452 85.147002) (end 104.14 87.501522) (width 0.25) (layer "F.Cu") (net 4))
 (segment (start 76.835 82.185) (end 76.565 81.915) (width 0.25) (layer "F.Cu") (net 4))
 (segment (start 80.22 75.1225) (end 76.6025 78.74) (width 0.25) (layer "F.Cu") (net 4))
 (segment (start 76.835 85.725) (end 76.835 82.185) (width 0.25) (layer "F.Cu") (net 4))
 (segment (start 105.011758 78.24) (end 106.095879 79.324121) (width 0.25) (layer "F.Cu") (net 4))
 (segment (start 106.49452 79.722763) (end 106.49452 83.82) (width 0.25) (layer "F.Cu") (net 4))
 (segment (start 104.14 87.501522) (end 104.14 87.63) (width 0.25) (layer "F.Cu") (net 4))
 (segment (start 106.095879 79.324121) (end 106.49452 79.722763) (width 0.25) (layer "F.Cu") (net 4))
 (segment (start 104.775 78.24) (end 105.011758 78.24) (width 0.25) (layer "F.Cu") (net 4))
 (segment (start 76.6025 81.8775) (end 76.565 81.915) (width 0.25) (layer "F.Cu") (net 4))
 (segment (start 106.49452 83.82) (end 106.49452 85.147002) (width 0.25) (layer "F.Cu") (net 4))
 (segment (start 76.6025 78.74) (end 76.6025 81.8775) (width 0.25) (layer "F.Cu") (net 4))
 (via (at 76.835 85.725) (size 0.8) (drill 0.4) (layers "F.Cu" "B.Cu") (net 4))
 (via (at 104.14 87.63) (size 0.8) (drill 0.4) (layers "F.Cu" "B.Cu") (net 4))
 (segment (start 95.885 87.63) (end 78.74 87.63) (width 0.25) (layer "B.Cu") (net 4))
 (segment (start 104.14 87.63) (end 95.885 87.63) (width 0.25) (layer "B.Cu") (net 4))
 (segment (start 78.74 87.63) (end 76.835 85.725) (width 0.25) (layer "B.Cu") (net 4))
 (segment (start 82.3575 77.6625) (end 80.01 80.01) (width 0.25) (layer "F.Cu") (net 2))
 (segment (start 103.545 76.24) (end 102.87 75.565) (width 0.25) (layer "F.Cu") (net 2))
 (segment (start 83.2 77.6625) (end 82.3575 77.6625) (width 0.25) (layer "F.Cu") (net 2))
 (segment (start 76.2 91.71) (end 80.01 91.71) (width 0.25) (layer "F.Cu") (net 2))
 (segment (start 104.775 76.24) (end 103.545 76.24) (width 0.25) (layer "F.Cu") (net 2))
 (segment (start 80.01 77.47) (end 80.01 80.01) (width 0.25) (layer "F.Cu") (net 2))
 (segment (start 80.01 87.9) (end 76.2 91.71) (width 0.25) (layer "F.Cu") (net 2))
 (segment (start 80.01 80.01) (end 80.01 87.9) (width 0.25) (layer "F.Cu") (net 2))
 (via (at 80.01 77.47) (size 0.8) (drill 0.4) (layers "F.Cu" "B.Cu") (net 2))
 (via (at 102.87 75.565) (size 0.8) (drill 0.4) (layers "F.Cu" "B.Cu") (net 2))
 (segment (start 81.915 75.565) (end 80.01 77.47) (width 0.25) (layer "B.Cu") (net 2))
 (segment (start 102.87 75.565) (end 81.915 75.565) (width 0.25) (layer "B.Cu") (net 2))
 (segment (start 101.162114 89.0925) (end 100.7 89.0925) (width 0.25) (layer "F.Cu") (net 5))
 (segment (start 104.775 79.24) (end 105.37604 79.24) (width 0.25) (layer "F.Cu") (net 5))
 (segment (start 105.37604 79.24) (end 106.045 79.90896) (width 0.25) (layer "F.Cu") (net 5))
 (segment (start 106.045 84.209614) (end 101.162114 89.0925) (width 0.25) (layer "F.Cu") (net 5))
 (segment (start 106.045 79.90896) (end 106.045 84.209614) (width 0.25) (layer "F.Cu") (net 5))
 (segment (start 101.7 77.6625) (end 102.87 78.8325) (width 0.25) (layer "F.Cu") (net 7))
 (segment (start 104.17396 81.24) (end 104.775 81.24) (width 0.25) (layer "F.Cu") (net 7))
 (segment (start 100.7 77.6625) (end 101.7 77.6625) (width 0.25) (layer "F.Cu") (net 7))
 (segment (start 102.87 78.8325) (end 102.87 79.93604) (width 0.25) (layer "F.Cu") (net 7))
 (segment (start 102.87 79.93604) (end 104.17396 81.24) (width 0.25) (layer "F.Cu") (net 7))
 (segment (start 101.7 76.3925) (end 104.025489 78.717989) (width 0.25) (layer "F.Cu") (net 6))
 (segment (start 104.025489 78.717989) (end 104.025489 79.895489) (width 0.25) (layer "F.Cu") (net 6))
 (segment (start 104.025489 79.895489) (end 104.37 80.24) (width 0.25) (layer "F.Cu") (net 6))
 (segment (start 104.37 80.24) (end 104.775 80.24) (width 0.25) (layer "F.Cu") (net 6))
 (segment (start 100.7 76.3925) (end 101.7 76.3925) (width 0.25) (layer "F.Cu") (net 6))
 (segment (start 69.335 81.28) (end 68.53548 82.07952) (width 0.25) (layer "F.Cu") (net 10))
 (segment (start 68.53548 86.61548) (end 69.26 87.34) (width 0.25) (layer "F.Cu") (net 10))
 (segment (start 68.53548 82.07952) (end 68.53548 86.61548) (width 0.25) (layer "F.Cu") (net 10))
 (segment (start 86.995 100.33) (end 83.82 97.155) (width 0.25) (layer "F.Cu") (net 11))
 (segment (start 72.025 97.155) (end 69.485 94.615) (width 0.25) (layer "F.Cu") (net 11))
 (segment (start 83.82 97.155) (end 72.025 97.155) (width 0.25) (layer "F.Cu") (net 11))
 (segment (start 88.2 100.33) (end 86.995 100.33) (width 0.25) (layer "F.Cu") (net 11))
 (segment (start 88.576072 101.6) (end 93.7615 96.414572) (width 0.25) (layer "F.Cu") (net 13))
 (segment (start 96.395 91.6165) (end 93.7615 94.25) (width 0.25) (layer "F.Cu") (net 13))
 (segment (start 93.7615 96.414572) (end 93.7615 94.25) (width 0.25) (layer "F.Cu") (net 13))
 (segment (start 88.2 101.6) (end 88.576072 101.6) (width 0.25) (layer "F.Cu") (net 13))
 (segment (start 96.395 90.6165) (end 96.395 91.6165) (width 0.25) (layer "F.Cu") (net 13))
 (segment (start 93.7615 94.25) (end 92.075 94.25) (width 0.25) (layer "F.Cu") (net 13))
 (segment (start 97.665 90.5925) (end 97.665 93.74) (width 0.25) (layer "F.Cu") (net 12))
 (segment (start 95.25 96.52) (end 95.25 95.25) (width 0.25) (layer "F.Cu") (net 12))
 (segment (start 96.25 94.25) (end 97.155 94.25) (width 0.25) (layer "F.Cu") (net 12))
 (segment (start 97.665 93.74) (end 97.155 94.25) (width 0.25) (layer "F.Cu") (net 12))
 (segment (start 88.2 102.87) (end 88.9 102.87) (width 0.25) (layer "F.Cu") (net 12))
 (segment (start 88.9 102.87) (end 95.25 96.52) (width 0.25) (layer "F.Cu") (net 12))
 (segment (start 95.25 95.25) (end 96.25 94.25) (width 0.25) (layer "F.Cu") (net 12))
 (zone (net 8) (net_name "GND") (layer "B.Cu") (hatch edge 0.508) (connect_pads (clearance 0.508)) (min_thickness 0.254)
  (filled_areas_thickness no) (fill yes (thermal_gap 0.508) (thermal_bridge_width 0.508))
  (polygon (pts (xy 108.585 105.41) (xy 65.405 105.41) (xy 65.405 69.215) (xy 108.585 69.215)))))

